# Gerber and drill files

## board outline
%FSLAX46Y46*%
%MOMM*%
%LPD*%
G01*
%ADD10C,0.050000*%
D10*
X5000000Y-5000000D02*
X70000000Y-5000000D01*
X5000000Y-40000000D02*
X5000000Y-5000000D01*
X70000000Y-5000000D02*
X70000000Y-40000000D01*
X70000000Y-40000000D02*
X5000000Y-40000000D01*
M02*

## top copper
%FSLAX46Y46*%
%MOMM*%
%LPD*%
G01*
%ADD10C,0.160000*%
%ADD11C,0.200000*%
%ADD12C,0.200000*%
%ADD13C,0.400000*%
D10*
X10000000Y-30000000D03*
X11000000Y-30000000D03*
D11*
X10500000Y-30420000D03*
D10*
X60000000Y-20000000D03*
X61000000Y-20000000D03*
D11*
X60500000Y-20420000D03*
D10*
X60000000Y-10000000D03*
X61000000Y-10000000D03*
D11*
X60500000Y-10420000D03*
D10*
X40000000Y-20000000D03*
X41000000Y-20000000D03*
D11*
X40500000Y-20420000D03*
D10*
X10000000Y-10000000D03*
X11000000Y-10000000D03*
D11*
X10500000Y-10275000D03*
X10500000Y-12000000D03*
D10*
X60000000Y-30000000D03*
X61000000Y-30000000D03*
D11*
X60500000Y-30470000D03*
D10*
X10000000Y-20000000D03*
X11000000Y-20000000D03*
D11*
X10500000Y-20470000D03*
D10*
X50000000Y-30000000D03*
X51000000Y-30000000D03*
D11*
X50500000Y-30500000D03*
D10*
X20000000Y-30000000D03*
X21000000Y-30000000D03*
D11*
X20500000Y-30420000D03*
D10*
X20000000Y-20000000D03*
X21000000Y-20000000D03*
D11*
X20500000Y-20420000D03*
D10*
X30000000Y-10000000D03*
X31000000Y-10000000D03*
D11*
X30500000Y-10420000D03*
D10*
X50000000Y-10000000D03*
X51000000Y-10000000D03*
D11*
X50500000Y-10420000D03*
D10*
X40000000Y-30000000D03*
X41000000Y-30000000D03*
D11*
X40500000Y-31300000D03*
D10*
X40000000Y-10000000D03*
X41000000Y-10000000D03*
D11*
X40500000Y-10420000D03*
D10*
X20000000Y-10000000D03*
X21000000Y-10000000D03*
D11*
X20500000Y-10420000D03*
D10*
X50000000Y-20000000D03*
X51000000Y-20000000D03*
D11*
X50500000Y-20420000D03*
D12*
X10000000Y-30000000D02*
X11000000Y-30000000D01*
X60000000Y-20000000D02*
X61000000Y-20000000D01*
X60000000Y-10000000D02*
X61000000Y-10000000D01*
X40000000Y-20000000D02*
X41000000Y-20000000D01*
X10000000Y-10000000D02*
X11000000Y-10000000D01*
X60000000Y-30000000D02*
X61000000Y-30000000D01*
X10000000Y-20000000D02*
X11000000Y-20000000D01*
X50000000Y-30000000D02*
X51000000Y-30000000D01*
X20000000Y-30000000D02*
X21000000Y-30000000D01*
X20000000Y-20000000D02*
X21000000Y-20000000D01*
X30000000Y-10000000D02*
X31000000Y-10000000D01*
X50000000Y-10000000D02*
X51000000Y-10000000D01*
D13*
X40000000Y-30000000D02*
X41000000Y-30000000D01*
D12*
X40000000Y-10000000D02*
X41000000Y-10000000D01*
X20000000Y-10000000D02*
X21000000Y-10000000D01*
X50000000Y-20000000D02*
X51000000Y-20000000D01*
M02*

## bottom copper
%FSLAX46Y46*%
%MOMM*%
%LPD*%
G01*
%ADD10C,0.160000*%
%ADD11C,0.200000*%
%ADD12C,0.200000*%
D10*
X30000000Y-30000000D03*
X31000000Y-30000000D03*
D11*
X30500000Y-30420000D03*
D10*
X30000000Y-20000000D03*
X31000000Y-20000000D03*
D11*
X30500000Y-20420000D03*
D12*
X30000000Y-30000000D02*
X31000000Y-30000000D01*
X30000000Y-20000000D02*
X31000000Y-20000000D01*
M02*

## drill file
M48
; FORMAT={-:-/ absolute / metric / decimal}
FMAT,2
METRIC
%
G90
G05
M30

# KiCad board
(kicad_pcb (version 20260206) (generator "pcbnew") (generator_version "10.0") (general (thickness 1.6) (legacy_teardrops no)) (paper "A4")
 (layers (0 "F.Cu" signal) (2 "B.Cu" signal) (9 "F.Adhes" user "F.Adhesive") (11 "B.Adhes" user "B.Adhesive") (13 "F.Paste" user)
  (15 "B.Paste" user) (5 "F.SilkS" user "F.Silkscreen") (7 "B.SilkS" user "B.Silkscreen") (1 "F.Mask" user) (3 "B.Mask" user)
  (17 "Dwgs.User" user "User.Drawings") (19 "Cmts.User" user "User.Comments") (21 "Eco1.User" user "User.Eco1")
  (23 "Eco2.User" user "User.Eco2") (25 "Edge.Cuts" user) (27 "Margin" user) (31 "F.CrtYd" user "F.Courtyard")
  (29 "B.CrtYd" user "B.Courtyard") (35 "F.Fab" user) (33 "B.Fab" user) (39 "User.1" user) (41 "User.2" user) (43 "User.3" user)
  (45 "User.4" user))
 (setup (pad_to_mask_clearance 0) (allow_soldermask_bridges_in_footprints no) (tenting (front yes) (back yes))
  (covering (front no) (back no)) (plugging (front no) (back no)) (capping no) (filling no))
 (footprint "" (layer "F.Cu") (at 10 30)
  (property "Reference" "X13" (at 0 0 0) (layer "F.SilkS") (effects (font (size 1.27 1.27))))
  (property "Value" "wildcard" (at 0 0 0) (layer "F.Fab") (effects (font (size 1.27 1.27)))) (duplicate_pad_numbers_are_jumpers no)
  (pad "1" smd circle (at 0 0) (size 0.16 0.16) (layers "F.Cu") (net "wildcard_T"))
  (pad "2" smd circle (at 1 0) (size 0.16 0.16) (layers "F.Cu") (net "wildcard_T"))
  (pad "3" smd circle (at 0.5 0.42) (size 0.2 0.2) (layers "F.Cu") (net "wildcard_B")))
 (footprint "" (layer "F.Cu") (at 60 20)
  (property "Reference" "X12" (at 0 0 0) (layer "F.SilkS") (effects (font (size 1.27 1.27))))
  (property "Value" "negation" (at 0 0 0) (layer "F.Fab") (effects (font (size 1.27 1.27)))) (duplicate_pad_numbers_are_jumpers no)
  (pad "1" smd circle (at 0 0) (size 0.16 0.16) (layers "F.Cu") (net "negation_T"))
  (pad "2" smd circle (at 1 0) (size 0.16 0.16) (layers "F.Cu") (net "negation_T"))
  (pad "3" smd circle (at 0.5 0.42) (size 0.2 0.2) (layers "F.Cu") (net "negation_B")))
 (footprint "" (layer "F.Cu") (at 60 10)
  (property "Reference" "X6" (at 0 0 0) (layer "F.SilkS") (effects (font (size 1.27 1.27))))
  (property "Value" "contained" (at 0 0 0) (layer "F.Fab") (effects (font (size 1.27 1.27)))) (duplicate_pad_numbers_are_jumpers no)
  (pad "1" smd circle (at 0 0) (size 0.16 0.16) (layers "F.Cu") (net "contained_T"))
  (pad "2" smd circle (at 1 0) (size 0.16 0.16) (layers "F.Cu") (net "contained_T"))
  (pad "3" smd circle (at 0.5 0.42) (size 0.2 0.2) (layers "F.Cu") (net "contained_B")))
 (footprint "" (layer "F.Cu") (at 40 20)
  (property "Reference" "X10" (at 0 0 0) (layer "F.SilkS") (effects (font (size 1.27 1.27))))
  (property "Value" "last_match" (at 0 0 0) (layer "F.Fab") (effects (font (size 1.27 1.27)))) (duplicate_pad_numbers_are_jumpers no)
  (pad "1" smd circle (at 0 0) (size 0.16 0.16) (layers "F.Cu") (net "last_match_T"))
  (pad "2" smd circle (at 1 0) (size 0.16 0.16) (layers "F.Cu") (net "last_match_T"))
  (pad "3" smd circle (at 0.5 0.42) (size 0.2 0.2) (layers "F.Cu") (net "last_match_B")))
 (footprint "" (layer "F.Cu") (at 10 10)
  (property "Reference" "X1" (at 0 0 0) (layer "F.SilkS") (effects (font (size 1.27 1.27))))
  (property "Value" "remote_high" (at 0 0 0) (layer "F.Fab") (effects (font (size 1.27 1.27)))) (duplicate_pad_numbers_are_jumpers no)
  (pad "1" smd circle (at 0 0) (size 0.16 0.16) (layers "F.Cu") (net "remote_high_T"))
  (pad "2" smd circle (at 1 0) (size 0.16 0.16) (layers "F.Cu") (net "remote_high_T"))
  (pad "3" smd circle (at 0.5 0.275) (size 0.2 0.2) (layers "F.Cu") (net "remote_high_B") (clearance 0.05))
  (pad "4" smd circle (at 0.5 2) (size 0.2 0.2) (layers "F.Cu") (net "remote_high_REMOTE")))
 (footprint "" (layer "F.Cu") (at 60 30)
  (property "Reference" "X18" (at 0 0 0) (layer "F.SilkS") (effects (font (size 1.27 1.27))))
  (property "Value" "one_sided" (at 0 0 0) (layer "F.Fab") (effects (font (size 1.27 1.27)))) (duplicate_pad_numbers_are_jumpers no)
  (pad "1" smd circle (at 0 0) (size 0.16 0.16) (layers "F.Cu") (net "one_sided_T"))
  (pad "2" smd circle (at 1 0) (size 0.16 0.16) (layers "F.Cu") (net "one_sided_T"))
  (pad "3" smd circle (at 0.5 0.47) (size 0.2 0.2) (layers "F.Cu") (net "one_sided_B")))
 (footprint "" (layer "F.Cu") (at 10 20)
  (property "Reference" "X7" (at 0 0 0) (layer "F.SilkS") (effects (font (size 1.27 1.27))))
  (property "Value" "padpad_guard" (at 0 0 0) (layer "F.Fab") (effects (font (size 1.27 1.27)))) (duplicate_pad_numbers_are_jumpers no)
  (pad "1" smd circle (at 0 0) (size 0.16 0.16) (layers "F.Cu") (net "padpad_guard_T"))
  (pad "2" smd circle (at 1 0) (size 0.16 0.16) (layers "F.Cu") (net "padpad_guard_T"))
  (pad "3" smd circle (at 0.5 0.47) (size 0.2 0.2) (layers "F.Cu") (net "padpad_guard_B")))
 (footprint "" (layer "F.Cu") (at 50 30)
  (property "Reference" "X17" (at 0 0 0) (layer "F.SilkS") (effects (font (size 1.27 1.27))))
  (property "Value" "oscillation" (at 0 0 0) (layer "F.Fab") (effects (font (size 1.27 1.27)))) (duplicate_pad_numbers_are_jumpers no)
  (pad "1" smd circle (at 0 0) (size 0.16 0.16) (layers "F.Cu") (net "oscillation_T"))
  (pad "2" smd circle (at 1 0) (size 0.16 0.16) (layers "F.Cu") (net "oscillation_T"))
  (pad "3" smd circle (at 0.5 0.5) (size 0.2 0.2) (layers "F.Cu") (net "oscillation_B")))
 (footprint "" (layer "F.Cu") (at 20 30)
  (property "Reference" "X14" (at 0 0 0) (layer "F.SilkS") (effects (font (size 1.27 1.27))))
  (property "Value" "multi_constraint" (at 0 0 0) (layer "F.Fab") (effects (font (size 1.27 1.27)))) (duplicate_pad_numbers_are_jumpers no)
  (pad "1" smd circle (at 0 0) (size 0.16 0.16) (layers "F.Cu") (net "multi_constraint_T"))
  (pad "2" smd circle (at 1 0) (size 0.16 0.16) (layers "F.Cu") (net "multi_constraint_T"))
  (pad "3" smd circle (at 0.5 0.42) (size 0.2 0.2) (layers "F.Cu") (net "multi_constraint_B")))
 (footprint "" (layer "F.Cu") (at 30 30)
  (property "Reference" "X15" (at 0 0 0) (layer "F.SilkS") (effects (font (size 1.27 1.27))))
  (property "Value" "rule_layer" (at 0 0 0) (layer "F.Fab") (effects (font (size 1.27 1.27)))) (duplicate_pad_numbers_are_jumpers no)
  (pad "1" smd circle (at 0 0) (size 0.16 0.16) (layers "B.Cu") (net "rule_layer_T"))
  (pad "2" smd circle (at 1 0) (size 0.16 0.16) (layers "B.Cu") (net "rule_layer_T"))
  (pad "3" smd circle (at 0.5 0.42) (size 0.2 0.2) (layers "B.Cu") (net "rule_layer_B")))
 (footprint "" (layer "F.Cu") (at 20 20)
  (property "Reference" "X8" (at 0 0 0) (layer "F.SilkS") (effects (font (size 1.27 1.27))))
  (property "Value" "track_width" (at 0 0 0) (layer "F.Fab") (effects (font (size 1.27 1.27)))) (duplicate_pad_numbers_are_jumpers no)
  (pad "1" smd circle (at 0 0) (size 0.16 0.16) (layers "F.Cu") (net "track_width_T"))
  (pad "2" smd circle (at 1 0) (size 0.16 0.16) (layers "F.Cu") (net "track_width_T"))
  (pad "3" smd circle (at 0.5 0.42) (size 0.2 0.2) (layers "F.Cu") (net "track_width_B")))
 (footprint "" (layer "F.Cu") (at 30 10)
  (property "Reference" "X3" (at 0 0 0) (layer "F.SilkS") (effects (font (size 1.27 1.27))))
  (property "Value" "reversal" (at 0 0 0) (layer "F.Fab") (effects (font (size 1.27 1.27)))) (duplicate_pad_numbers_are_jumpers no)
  (pad "1" smd circle (at 0 0) (size 0.16 0.16) (layers "F.Cu") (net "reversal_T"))
  (pad "2" smd circle (at 1 0) (size 0.16 0.16) (layers "F.Cu") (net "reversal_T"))
  (pad "3" smd circle (at 0.5 0.42) (size 0.2 0.2) (layers "F.Cu") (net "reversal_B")))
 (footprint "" (layer "F.Cu") (at 50 10)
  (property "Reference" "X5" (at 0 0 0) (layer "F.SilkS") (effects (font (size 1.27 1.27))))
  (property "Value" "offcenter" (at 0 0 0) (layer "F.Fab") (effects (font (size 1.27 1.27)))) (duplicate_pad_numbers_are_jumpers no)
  (pad "1" smd circle (at 0 0) (size 0.16 0.16) (layers "F.Cu") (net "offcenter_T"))
  (pad "2" smd circle (at 1 0) (size 0.16 0.16) (layers "F.Cu") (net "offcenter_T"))
  (pad "3" smd circle (at 0.5 0.42) (size 0.2 0.2) (layers "F.Cu") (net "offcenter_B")))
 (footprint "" (layer "F.Cu") (at 40 30)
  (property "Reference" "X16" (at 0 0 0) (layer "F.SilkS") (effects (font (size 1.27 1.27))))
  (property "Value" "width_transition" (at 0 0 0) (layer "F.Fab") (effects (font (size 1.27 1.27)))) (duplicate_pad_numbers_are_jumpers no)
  (pad "1" smd circle (at 0 0) (size 0.16 0.16) (layers "F.Cu") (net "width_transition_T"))
  (pad "2" smd circle (at 1 0) (size 0.16 0.16) (layers "F.Cu") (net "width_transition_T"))
  (pad "3" smd circle (at 0.5 1.3) (size 0.2 0.2) (layers "F.Cu") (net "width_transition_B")))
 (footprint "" (layer "F.Cu") (at 30 20)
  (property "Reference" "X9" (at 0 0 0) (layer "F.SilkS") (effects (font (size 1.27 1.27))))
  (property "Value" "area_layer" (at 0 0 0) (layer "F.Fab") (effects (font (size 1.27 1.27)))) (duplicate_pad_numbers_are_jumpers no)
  (pad "1" smd circle (at 0 0) (size 0.16 0.16) (layers "B.Cu") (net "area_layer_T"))
  (pad "2" smd circle (at 1 0) (size 0.16 0.16) (layers "B.Cu") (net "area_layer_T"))
  (pad "3" smd circle (at 0.5 0.42) (size 0.2 0.2) (layers "B.Cu") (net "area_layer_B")))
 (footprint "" (layer "F.Cu") (at 40 10)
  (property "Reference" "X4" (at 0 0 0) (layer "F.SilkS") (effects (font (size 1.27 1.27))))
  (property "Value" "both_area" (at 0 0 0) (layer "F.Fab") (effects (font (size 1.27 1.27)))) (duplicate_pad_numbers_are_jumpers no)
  (pad "1" smd circle (at 0 0) (size 0.16 0.16) (layers "F.Cu") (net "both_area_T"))
  (pad "2" smd circle (at 1 0) (size 0.16 0.16) (layers "F.Cu") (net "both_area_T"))
  (pad "3" smd circle (at 0.5 0.42) (size 0.2 0.2) (layers "F.Cu") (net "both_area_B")))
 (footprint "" (layer "F.Cu") (at 20 10)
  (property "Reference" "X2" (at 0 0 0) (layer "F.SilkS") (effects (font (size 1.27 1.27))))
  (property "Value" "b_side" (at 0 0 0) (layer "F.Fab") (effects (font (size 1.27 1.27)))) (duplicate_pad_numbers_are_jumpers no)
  (pad "1" smd circle (at 0 0) (size 0.16 0.16) (layers "F.Cu") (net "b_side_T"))
  (pad "2" smd circle (at 1 0) (size 0.16 0.16) (layers "F.Cu") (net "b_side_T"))
  (pad "3" smd circle (at 0.5 0.42) (size 0.2 0.2) (layers "F.Cu") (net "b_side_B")))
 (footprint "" (layer "F.Cu") (at 50 20)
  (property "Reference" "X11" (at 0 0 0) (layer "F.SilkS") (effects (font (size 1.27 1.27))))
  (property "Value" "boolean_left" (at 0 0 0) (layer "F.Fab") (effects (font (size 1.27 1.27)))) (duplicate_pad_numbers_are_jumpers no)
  (pad "1" smd circle (at 0 0) (size 0.16 0.16) (layers "F.Cu") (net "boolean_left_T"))
  (pad "2" smd circle (at 1 0) (size 0.16 0.16) (layers "F.Cu") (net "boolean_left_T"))
  (pad "3" smd circle (at 0.5 0.42) (size 0.2 0.2) (layers "F.Cu") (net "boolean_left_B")))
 (gr_line (start 5 5) (end 70 5) (stroke (width 0.05) (type default)) (layer "Edge.Cuts"))
 (gr_line (start 5 40) (end 5 5) (stroke (width 0.05) (type default)) (layer "Edge.Cuts"))
 (gr_line (start 70 5) (end 70 40) (stroke (width 0.05) (type default)) (layer "Edge.Cuts"))
 (gr_line (start 70 40) (end 5 40) (stroke (width 0.05) (type default)) (layer "Edge.Cuts"))
 (segment (start 10 30) (end 11 30) (width 0.2) (layer "F.Cu") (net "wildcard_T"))
 (segment (start 60 20) (end 61 20) (width 0.2) (layer "F.Cu") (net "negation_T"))
 (segment (start 60 10) (end 61 10) (width 0.2) (layer "F.Cu") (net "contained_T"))
 (segment (start 40 20) (end 41 20) (width 0.2) (layer "F.Cu") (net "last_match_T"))
 (segment (start 10 10) (end 11 10) (width 0.2) (layer "F.Cu") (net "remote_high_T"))
 (segment (start 60 30) (end 61 30) (width 0.2) (layer "F.Cu") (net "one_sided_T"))
 (segment (start 10 20) (end 11 20) (width 0.2) (layer "F.Cu") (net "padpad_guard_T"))
 (segment (start 50 30) (end 51 30) (width 0.2) (layer "F.Cu") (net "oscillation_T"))
 (segment (start 20 30) (end 21 30) (width 0.2) (layer "F.Cu") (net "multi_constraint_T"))
 (segment (start 30 30) (end 31 30) (width 0.2) (layer "B.Cu") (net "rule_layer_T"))
 (segment (start 20 20) (end 21 20) (width 0.2) (layer "F.Cu") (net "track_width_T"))
 (segment (start 30 10) (end 31 10) (width 0.2) (layer "F.Cu") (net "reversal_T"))
 (segment (start 50 10) (end 51 10) (width 0.2) (layer "F.Cu") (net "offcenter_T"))
 (segment (start 40 30) (end 41 30) (width 0.4) (layer "F.Cu") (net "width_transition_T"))
 (segment (start 30 20) (end 31 20) (width 0.2) (layer "B.Cu") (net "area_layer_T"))
 (segment (start 40 10) (end 41 10) (width 0.2) (layer "F.Cu") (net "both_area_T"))
 (segment (start 20 10) (end 21 10) (width 0.2) (layer "F.Cu") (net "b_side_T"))
 (segment (start 50 20) (end 51 20) (width 0.2) (layer "F.Cu") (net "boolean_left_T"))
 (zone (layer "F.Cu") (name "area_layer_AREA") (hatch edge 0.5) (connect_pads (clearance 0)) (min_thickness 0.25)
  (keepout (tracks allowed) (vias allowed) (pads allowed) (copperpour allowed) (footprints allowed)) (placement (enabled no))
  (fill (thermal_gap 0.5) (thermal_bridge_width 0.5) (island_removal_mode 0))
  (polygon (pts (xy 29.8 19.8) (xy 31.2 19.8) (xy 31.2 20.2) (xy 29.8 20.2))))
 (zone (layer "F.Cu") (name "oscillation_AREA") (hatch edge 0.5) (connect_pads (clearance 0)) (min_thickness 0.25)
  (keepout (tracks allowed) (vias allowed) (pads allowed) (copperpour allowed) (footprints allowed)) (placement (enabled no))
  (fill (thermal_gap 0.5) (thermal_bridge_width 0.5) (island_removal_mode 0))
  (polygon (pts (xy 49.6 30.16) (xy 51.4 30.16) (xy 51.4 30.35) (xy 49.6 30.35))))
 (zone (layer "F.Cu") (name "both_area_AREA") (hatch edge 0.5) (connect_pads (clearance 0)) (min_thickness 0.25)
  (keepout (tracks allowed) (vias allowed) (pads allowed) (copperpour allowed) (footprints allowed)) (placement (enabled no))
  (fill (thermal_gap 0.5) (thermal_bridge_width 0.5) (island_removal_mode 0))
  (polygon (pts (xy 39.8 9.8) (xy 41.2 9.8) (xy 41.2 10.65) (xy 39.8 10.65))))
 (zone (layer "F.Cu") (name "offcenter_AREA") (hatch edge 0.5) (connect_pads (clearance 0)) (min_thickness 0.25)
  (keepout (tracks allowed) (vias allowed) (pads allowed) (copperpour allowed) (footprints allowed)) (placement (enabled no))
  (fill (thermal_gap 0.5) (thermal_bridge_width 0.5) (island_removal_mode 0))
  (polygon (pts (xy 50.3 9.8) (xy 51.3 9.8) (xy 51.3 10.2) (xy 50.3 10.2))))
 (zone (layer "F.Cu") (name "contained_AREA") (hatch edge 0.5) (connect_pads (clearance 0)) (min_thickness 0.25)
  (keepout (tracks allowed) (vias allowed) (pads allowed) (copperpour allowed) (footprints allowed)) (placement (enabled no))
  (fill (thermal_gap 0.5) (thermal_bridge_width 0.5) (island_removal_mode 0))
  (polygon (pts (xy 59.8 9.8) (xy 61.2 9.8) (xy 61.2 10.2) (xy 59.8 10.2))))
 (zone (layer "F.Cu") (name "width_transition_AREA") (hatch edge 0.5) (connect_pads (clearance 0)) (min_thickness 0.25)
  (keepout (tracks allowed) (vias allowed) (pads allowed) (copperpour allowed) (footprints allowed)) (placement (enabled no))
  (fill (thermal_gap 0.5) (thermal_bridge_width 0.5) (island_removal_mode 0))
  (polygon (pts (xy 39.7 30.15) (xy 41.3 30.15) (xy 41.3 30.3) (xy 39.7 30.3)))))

